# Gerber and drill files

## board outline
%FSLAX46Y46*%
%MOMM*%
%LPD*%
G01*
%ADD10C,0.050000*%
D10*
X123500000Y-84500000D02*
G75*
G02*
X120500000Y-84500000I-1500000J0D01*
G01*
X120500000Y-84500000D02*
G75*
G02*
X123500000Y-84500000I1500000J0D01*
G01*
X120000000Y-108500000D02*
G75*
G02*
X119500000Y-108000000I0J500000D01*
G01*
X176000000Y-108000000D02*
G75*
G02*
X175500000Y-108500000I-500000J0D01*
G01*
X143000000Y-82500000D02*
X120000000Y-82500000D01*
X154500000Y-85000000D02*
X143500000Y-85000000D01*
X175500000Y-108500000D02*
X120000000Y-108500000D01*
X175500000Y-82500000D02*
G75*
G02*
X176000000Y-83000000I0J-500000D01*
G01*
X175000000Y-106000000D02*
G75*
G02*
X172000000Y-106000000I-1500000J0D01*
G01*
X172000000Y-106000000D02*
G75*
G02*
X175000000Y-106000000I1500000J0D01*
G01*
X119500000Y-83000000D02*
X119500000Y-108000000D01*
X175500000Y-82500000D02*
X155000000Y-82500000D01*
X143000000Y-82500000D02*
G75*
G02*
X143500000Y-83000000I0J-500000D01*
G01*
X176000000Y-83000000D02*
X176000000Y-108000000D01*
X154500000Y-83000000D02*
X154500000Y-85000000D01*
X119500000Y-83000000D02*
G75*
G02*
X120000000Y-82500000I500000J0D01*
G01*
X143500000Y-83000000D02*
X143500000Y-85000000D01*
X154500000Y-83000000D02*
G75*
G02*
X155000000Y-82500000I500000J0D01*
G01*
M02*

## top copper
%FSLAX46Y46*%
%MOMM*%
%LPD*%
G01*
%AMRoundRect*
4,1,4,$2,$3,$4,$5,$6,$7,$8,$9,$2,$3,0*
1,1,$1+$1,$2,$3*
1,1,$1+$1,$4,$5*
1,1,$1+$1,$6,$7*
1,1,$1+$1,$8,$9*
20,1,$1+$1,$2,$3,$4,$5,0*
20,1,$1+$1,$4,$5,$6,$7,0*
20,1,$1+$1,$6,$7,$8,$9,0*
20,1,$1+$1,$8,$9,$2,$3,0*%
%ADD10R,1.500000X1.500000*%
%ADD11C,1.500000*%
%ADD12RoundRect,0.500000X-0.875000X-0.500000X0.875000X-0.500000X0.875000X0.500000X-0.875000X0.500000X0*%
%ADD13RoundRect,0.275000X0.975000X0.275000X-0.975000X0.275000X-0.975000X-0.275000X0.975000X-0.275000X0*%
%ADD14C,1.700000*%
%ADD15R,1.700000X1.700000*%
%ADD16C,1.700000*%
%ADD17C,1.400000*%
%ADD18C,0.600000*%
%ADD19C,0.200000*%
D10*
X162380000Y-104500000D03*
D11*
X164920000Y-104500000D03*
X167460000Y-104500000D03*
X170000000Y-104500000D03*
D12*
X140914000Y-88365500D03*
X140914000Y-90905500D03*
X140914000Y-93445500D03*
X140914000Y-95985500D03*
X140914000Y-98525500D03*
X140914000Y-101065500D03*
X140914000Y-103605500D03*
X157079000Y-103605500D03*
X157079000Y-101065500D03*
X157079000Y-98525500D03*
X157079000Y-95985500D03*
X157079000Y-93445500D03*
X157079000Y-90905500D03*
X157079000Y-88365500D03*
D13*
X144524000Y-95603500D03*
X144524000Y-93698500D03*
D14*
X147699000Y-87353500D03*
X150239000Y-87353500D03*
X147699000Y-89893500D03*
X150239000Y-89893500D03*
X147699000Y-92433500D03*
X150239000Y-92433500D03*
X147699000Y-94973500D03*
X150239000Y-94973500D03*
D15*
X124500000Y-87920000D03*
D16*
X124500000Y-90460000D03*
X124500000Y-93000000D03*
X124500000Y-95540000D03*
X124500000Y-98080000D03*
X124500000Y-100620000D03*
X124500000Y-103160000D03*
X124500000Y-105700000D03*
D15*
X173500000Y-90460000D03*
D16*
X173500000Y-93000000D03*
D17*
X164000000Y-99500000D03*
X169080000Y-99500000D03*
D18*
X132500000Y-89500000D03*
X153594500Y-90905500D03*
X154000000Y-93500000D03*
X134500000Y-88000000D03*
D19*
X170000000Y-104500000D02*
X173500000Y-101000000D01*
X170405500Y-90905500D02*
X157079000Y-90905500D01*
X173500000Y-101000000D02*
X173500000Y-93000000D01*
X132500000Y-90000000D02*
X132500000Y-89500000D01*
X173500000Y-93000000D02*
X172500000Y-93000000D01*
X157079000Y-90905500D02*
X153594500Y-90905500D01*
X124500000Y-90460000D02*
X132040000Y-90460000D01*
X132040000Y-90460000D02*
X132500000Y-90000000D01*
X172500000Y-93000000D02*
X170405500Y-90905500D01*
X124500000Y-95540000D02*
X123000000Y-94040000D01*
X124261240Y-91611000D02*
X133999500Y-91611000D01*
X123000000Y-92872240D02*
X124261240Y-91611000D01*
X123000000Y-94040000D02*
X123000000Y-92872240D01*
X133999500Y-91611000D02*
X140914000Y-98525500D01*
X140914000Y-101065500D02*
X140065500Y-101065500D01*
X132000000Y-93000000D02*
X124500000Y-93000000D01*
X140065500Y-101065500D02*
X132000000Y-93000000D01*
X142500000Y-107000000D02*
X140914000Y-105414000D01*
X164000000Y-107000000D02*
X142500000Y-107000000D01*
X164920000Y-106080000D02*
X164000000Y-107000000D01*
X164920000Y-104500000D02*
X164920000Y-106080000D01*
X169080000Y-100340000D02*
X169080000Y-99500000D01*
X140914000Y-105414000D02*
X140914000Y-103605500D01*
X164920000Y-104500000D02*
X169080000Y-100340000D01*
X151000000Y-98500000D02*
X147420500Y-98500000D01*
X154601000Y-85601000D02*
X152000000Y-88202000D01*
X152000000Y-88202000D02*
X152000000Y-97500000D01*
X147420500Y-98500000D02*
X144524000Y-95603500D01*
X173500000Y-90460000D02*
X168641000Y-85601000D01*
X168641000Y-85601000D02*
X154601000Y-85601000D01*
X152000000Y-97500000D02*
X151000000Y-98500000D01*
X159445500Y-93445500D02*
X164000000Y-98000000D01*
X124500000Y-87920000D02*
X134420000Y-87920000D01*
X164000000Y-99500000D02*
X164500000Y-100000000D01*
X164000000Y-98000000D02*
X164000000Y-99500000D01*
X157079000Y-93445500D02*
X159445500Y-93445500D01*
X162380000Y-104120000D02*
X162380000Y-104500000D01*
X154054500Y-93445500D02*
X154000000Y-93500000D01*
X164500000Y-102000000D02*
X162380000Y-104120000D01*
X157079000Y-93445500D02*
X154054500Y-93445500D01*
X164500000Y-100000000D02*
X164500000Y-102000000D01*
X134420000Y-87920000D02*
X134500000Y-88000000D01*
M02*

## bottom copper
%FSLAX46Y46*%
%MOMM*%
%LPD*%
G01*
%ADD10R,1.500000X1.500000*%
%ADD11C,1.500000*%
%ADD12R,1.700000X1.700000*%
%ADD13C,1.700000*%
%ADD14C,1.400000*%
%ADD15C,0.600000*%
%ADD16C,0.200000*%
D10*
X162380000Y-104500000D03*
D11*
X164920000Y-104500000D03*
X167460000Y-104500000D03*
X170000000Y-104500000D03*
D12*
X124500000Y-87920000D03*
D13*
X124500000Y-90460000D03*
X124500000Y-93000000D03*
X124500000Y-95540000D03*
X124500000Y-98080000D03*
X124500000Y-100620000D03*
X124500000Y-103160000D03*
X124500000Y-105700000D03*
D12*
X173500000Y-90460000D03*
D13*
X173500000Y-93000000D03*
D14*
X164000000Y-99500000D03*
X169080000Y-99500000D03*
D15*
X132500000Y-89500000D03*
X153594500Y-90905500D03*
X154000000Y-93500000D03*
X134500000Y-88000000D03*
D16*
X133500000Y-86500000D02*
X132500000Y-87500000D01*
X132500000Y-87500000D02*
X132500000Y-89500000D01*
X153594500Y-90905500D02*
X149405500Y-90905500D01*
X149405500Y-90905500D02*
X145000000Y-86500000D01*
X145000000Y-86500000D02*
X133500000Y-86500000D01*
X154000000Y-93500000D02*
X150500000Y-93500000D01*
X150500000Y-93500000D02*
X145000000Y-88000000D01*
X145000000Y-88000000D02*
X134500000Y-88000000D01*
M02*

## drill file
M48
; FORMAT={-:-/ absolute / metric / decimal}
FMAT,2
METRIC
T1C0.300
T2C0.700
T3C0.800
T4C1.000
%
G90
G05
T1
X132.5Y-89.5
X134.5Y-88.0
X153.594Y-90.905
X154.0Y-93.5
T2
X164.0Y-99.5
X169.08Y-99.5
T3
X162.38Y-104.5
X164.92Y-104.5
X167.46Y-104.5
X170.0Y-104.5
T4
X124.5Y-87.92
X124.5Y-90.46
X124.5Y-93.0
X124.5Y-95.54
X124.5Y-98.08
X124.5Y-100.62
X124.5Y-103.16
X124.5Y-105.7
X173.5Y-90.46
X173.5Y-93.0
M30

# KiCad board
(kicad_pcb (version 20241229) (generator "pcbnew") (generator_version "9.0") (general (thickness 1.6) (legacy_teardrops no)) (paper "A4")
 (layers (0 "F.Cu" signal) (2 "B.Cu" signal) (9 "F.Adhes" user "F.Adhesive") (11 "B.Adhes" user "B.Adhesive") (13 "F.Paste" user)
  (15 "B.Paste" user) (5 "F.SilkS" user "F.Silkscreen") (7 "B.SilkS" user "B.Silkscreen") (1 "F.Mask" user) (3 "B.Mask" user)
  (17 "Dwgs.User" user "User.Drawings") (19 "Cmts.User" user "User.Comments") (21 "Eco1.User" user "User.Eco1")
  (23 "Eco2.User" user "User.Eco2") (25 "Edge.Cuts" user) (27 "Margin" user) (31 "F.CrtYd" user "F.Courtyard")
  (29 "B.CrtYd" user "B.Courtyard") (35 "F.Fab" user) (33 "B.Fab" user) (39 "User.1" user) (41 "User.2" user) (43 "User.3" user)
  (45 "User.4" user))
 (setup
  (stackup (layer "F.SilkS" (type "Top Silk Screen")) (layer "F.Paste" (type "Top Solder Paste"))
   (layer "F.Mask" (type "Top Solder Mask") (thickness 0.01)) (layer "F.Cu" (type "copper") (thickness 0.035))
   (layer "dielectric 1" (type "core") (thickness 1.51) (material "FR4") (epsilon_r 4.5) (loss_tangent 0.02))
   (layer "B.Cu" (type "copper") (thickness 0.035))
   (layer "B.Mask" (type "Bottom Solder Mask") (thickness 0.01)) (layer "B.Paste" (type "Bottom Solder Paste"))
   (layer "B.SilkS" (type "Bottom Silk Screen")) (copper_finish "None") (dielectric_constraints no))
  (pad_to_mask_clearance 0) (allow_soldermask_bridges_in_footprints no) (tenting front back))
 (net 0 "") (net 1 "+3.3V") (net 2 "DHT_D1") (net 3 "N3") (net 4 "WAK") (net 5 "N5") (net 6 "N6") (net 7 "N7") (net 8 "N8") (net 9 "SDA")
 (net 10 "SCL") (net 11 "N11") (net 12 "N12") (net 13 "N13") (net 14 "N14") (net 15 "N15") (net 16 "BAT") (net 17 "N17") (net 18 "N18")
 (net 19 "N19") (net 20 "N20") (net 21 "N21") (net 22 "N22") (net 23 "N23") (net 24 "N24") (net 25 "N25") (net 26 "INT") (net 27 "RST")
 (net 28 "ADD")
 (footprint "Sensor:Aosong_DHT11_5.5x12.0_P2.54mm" (layer "F.Cu") (at 162.38 104.5 90)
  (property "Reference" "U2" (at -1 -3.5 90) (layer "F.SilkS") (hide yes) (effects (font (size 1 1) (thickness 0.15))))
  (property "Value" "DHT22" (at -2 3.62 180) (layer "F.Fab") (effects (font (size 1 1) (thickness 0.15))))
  (pad "1" thru_hole rect (at 0 0 90) (size 1.5 1.5) (drill 0.8) (layers "*.Cu" "*.Mask") (remove_unused_layers no) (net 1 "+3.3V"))
  (pad "2" thru_hole circle (at 0 2.54 90) (size 1.5 1.5) (drill 0.8) (layers "*.Cu" "*.Mask") (remove_unused_layers no) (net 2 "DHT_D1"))
  (pad "3" thru_hole circle (at 0 5.08 90) (size 1.5 1.5) (drill 0.8) (layers "*.Cu" "*.Mask") (remove_unused_layers no) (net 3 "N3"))
  (pad "4" thru_hole circle (at 0 7.62 90) (size 1.5 1.5) (drill 0.8) (layers "*.Cu" "*.Mask") (remove_unused_layers no) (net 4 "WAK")))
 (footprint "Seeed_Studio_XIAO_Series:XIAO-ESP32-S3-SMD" (layer "F.Cu") (at 140.079 106.4855)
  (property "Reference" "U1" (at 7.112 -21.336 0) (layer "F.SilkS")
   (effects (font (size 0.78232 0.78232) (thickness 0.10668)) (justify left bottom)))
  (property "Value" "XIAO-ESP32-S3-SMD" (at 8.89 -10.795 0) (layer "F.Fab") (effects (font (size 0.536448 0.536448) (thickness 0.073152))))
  (pad "1" smd roundrect (at 0.835 -18.12) (size 2.75 2) (layers "F.Cu" "F.Mask" "F.Paste") (roundrect_rratio 0.25) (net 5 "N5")
   (solder_mask_margin 0.0508) (thermal_bridge_angle 45))
  (pad "2" smd roundrect (at 0.835 -15.58) (size 2.75 2) (layers "F.Cu" "F.Mask" "F.Paste") (roundrect_rratio 0.25) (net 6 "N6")
   (solder_mask_margin 0.0508) (thermal_bridge_angle 45))
  (pad "3" smd roundrect (at 0.835 -13.04) (size 2.75 2) (layers "F.Cu" "F.Mask" "F.Paste") (roundrect_rratio 0.25) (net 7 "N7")
   (solder_mask_margin 0.0508) (thermal_bridge_angle 45))
  (pad "4" smd roundrect (at 0.835 -10.5) (size 2.75 2) (layers "F.Cu" "F.Mask" "F.Paste") (roundrect_rratio 0.25) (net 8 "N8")
   (solder_mask_margin 0.0508) (thermal_bridge_angle 45))
  (pad "5" smd roundrect (at 0.835 -7.96) (size 2.75 2) (layers "F.Cu" "F.Mask" "F.Paste") (roundrect_rratio 0.25) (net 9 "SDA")
   (solder_mask_margin 0.0508) (thermal_bridge_angle 45))
  (pad "6" smd roundrect (at 0.835 -5.42) (size 2.75 2) (layers "F.Cu" "F.Mask" "F.Paste") (roundrect_rratio 0.25) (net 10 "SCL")
   (solder_mask_margin 0.0508) (thermal_bridge_angle 45))
  (pad "7" smd roundrect (at 0.835 -2.88) (size 2.75 2) (layers "F.Cu" "F.Mask" "F.Paste") (roundrect_rratio 0.25) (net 2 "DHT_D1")
   (solder_mask_margin 0.0508) (thermal_bridge_angle 45))
  (pad "8" smd roundrect (at 17 -2.88) (size 2.75 2) (layers "F.Cu" "F.Mask" "F.Paste") (roundrect_rratio 0.25) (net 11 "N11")
   (solder_mask_margin 0.0508) (thermal_bridge_angle 45))
  (pad "9" smd roundrect (at 17 -5.42) (size 2.75 2) (layers "F.Cu" "F.Mask" "F.Paste") (roundrect_rratio 0.25) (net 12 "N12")
   (solder_mask_margin 0.0508) (thermal_bridge_angle 45))
  (pad "10" smd roundrect (at 17 -7.96) (size 2.75 2) (layers "F.Cu" "F.Mask" "F.Paste") (roundrect_rratio 0.25) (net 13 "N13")
   (solder_mask_margin 0.0508) (thermal_bridge_angle 45))
  (pad "11" smd roundrect (at 17 -10.5) (size 2.75 2) (layers "F.Cu" "F.Mask" "F.Paste") (roundrect_rratio 0.25) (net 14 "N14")
   (solder_mask_margin 0.0508) (thermal_bridge_angle 45))
  (pad "12" smd roundrect (at 17 -13.04) (size 2.75 2) (layers "F.Cu" "F.Mask" "F.Paste") (roundrect_rratio 0.25) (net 1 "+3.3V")
   (solder_mask_margin 0.0508) (thermal_bridge_angle 45))
  (pad "13" smd roundrect (at 17 -15.58) (size 2.75 2) (layers "F.Cu" "F.Mask" "F.Paste") (roundrect_rratio 0.25) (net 4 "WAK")
   (solder_mask_margin 0.0508) (thermal_bridge_angle 45))
  (pad "14" smd roundrect (at 17 -18.12) (size 2.75 2) (layers "F.Cu" "F.Mask" "F.Paste") (roundrect_rratio 0.25) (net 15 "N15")
   (solder_mask_margin 0.0508) (thermal_bridge_angle 45))
  (pad "15" smd roundrect (at 4.445 -10.882 180) (size 2.5 1.1) (layers "F.Cu" "F.Mask" "F.Paste") (roundrect_rratio 0.25) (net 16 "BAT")
   (solder_mask_margin 0.0508) (thermal_bridge_angle 45))
  (pad "16" smd roundrect (at 4.445 -12.787 180) (size 2.5 1.1) (layers "F.Cu" "F.Mask" "F.Paste") (roundrect_rratio 0.25) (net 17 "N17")
   (solder_mask_margin 0.0508) (thermal_bridge_angle 45))
  (pad "17" smd circle (at 7.62 -19.132) (size 1.7 1.7) (layers "F.Cu" "F.Mask" "F.Paste") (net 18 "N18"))
  (pad "18" smd circle (at 10.16 -19.132) (size 1.7 1.7) (layers "F.Cu" "F.Mask" "F.Paste") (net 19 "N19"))
  (pad "19" smd circle (at 7.62 -16.592) (size 1.7 1.7) (layers "F.Cu" "F.Mask" "F.Paste") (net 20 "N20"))
  (pad "20" smd circle (at 10.16 -16.592) (size 1.7 1.7) (layers "F.Cu" "F.Mask" "F.Paste") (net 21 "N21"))
  (pad "21" smd circle (at 7.62 -14.052) (size 1.7 1.7) (layers "F.Cu" "F.Mask" "F.Paste") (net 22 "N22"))
  (pad "22" smd circle (at 10.16 -14.052) (size 1.7 1.7) (layers "F.Cu" "F.Mask" "F.Paste") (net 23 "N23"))
  (pad "23" smd circle (at 7.62 -11.512) (size 1.7 1.7) (layers "F.Cu" "F.Mask" "F.Paste") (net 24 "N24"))
  (pad "24" smd circle (at 10.16 -11.512) (size 1.7 1.7) (layers "F.Cu" "F.Mask" "F.Paste") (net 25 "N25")))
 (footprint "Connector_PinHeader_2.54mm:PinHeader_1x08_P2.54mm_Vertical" (layer "F.Cu") (at 124.5 87.92)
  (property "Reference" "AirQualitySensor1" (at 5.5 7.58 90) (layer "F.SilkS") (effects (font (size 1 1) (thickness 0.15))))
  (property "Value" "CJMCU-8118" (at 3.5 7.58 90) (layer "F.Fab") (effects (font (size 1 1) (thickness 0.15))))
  (pad "1" thru_hole rect (at 0 0) (size 1.7 1.7) (drill 1) (layers "*.Cu" "*.Mask") (remove_unused_layers no) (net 1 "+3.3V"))
  (pad "2" thru_hole circle (at 0 2.54) (size 1.7 1.7) (drill 1) (layers "*.Cu" "*.Mask") (remove_unused_layers no) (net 4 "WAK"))
  (pad "3" thru_hole circle (at 0 5.08) (size 1.7 1.7) (drill 1) (layers "*.Cu" "*.Mask") (remove_unused_layers no) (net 10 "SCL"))
  (pad "4" thru_hole circle (at 0 7.62) (size 1.7 1.7) (drill 1) (layers "*.Cu" "*.Mask") (remove_unused_layers no) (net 9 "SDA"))
  (pad "5" thru_hole circle (at 0 10.16) (size 1.7 1.7) (drill 1) (layers "*.Cu" "*.Mask") (remove_unused_layers no) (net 4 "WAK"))
  (pad "6" thru_hole circle (at 0 12.7) (size 1.7 1.7) (drill 1) (layers "*.Cu" "*.Mask") (remove_unused_layers no) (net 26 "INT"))
  (pad "7" thru_hole circle (at 0 15.24) (size 1.7 1.7) (drill 1) (layers "*.Cu" "*.Mask") (remove_unused_layers no) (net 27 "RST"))
  (pad "8" thru_hole circle (at 0 17.78) (size 1.7 1.7) (drill 1) (layers "*.Cu" "*.Mask") (remove_unused_layers no) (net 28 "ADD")))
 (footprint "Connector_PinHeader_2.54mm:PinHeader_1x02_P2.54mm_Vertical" (layer "B.Cu") (at 173.5 90.46 180)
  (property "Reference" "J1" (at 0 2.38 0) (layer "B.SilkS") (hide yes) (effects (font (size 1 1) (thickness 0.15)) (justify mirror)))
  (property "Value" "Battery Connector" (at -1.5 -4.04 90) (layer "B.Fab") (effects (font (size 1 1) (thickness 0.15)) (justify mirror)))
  (pad "1" thru_hole rect (at 0 0 180) (size 1.7 1.7) (drill 1) (layers "*.Cu" "*.Mask") (remove_unused_layers no) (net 16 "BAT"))
  (pad "2" thru_hole circle (at 0 -2.54 180) (size 1.7 1.7) (drill 1) (layers "*.Cu" "*.Mask") (remove_unused_layers no) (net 4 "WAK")))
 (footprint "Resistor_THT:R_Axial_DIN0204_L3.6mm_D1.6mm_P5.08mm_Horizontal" (layer "B.Cu") (at 164 99.5)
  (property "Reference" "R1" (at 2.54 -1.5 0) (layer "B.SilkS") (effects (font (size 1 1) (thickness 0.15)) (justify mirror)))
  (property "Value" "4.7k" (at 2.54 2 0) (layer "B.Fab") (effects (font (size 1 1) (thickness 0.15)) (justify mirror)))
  (pad "1" thru_hole circle (at 0 0) (size 1.4 1.4) (drill 0.7) (layers "*.Cu" "*.Mask") (remove_unused_layers no) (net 1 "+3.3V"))
  (pad "2" thru_hole circle (at 5.08 0) (size 1.4 1.4) (drill 0.7) (layers "*.Cu" "*.Mask") (remove_unused_layers no) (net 2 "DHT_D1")))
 (gr_circle (center 122 84.5) (end 123.5 84.5) (stroke (width 0.05) (type solid)) (fill no) (layer "Edge.Cuts"))
 (gr_arc (start 120 108.5) (mid 119.646447 108.353553) (end 119.5 108) (stroke (width 0.05) (type default)) (layer "Edge.Cuts"))
 (gr_arc (start 176 108) (mid 175.853553 108.353553) (end 175.5 108.5) (stroke (width 0.05) (type default)) (layer "Edge.Cuts"))
 (gr_line (start 143 82.5) (end 120 82.5) (stroke (width 0.05) (type default)) (layer "Edge.Cuts"))
 (gr_line (start 154.5 85) (end 143.5 85) (stroke (width 0.05) (type default)) (layer "Edge.Cuts"))
 (gr_line (start 175.5 108.5) (end 120 108.5) (stroke (width 0.05) (type default)) (layer "Edge.Cuts"))
 (gr_arc (start 175.5 82.5) (mid 175.853553 82.646447) (end 176 83) (stroke (width 0.05) (type default)) (layer "Edge.Cuts"))
 (gr_circle (center 173.5 106) (end 175 106) (stroke (width 0.05) (type solid)) (fill no) (layer "Edge.Cuts"))
 (gr_line (start 119.5 83) (end 119.5 108) (stroke (width 0.05) (type default)) (layer "Edge.Cuts"))
 (gr_line (start 175.5 82.5) (end 155 82.5) (stroke (width 0.05) (type default)) (layer "Edge.Cuts"))
 (gr_arc (start 143 82.5) (mid 143.353553 82.646447) (end 143.5 83) (stroke (width 0.05) (type default)) (layer "Edge.Cuts"))
 (gr_line (start 176 83) (end 176 108) (stroke (width 0.05) (type default)) (layer "Edge.Cuts"))
 (gr_line (start 154.5 83) (end 154.5 85) (stroke (width 0.05) (type default)) (layer "Edge.Cuts"))
 (gr_arc (start 119.5 83) (mid 119.646447 82.646447) (end 120 82.5) (stroke (width 0.05) (type default)) (layer "Edge.Cuts"))
 (gr_line (start 143.5 83) (end 143.5 85) (stroke (width 0.05) (type default)) (layer "Edge.Cuts"))
 (gr_arc (start 154.5 83) (mid 154.646447 82.646447) (end 155 82.5) (stroke (width 0.05) (type default)) (layer "Edge.Cuts"))
 (segment (start 170 104.5) (end 173.5 101) (width 0.2) (layer "F.Cu") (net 4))
 (segment (start 170.4055 90.9055) (end 157.079 90.9055) (width 0.2) (layer "F.Cu") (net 4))
 (segment (start 173.5 101) (end 173.5 93) (width 0.2) (layer "F.Cu") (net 4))
 (segment (start 132.5 90) (end 132.5 89.5) (width 0.2) (layer "F.Cu") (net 4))
 (segment (start 173.5 93) (end 172.5 93) (width 0.2) (layer "F.Cu") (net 4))
 (segment (start 157.079 90.9055) (end 153.5945 90.9055) (width 0.2) (layer "F.Cu") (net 4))
 (segment (start 124.5 90.46) (end 132.04 90.46) (width 0.2) (layer "F.Cu") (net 4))
 (segment (start 132.04 90.46) (end 132.5 90) (width 0.2) (layer "F.Cu") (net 4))
 (segment (start 172.5 93) (end 170.4055 90.9055) (width 0.2) (layer "F.Cu") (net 4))
 (via (at 132.5 89.5) (size 0.6) (drill 0.3) (layers "F.Cu" "B.Cu") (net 4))
 (via (at 153.5945 90.9055) (size 0.6) (drill 0.3) (layers "F.Cu" "B.Cu") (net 4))
 (segment (start 133.5 86.5) (end 132.5 87.5) (width 0.2) (layer "B.Cu") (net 4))
 (segment (start 132.5 87.5) (end 132.5 89.5) (width 0.2) (layer "B.Cu") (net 4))
 (segment (start 153.5945 90.9055) (end 149.4055 90.9055) (width 0.2) (layer "B.Cu") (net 4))
 (segment (start 149.4055 90.9055) (end 145 86.5) (width 0.2) (layer "B.Cu") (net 4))
 (segment (start 145 86.5) (end 133.5 86.5) (width 0.2) (layer "B.Cu") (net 4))
 (segment (start 124.5 95.54) (end 123 94.04) (width 0.2) (layer "F.Cu") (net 9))
 (segment (start 124.26124 91.611) (end 133.9995 91.611) (width 0.2) (layer "F.Cu") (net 9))
 (segment (start 123 92.87224) (end 124.26124 91.611) (width 0.2) (layer "F.Cu") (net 9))
 (segment (start 123 94.04) (end 123 92.87224) (width 0.2) (layer "F.Cu") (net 9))
 (segment (start 133.9995 91.611) (end 140.914 98.5255) (width 0.2) (layer "F.Cu") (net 9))
 (segment (start 140.914 101.0655) (end 140.0655 101.0655) (width 0.2) (layer "F.Cu") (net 10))
 (segment (start 132 93) (end 124.5 93) (width 0.2) (layer "F.Cu") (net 10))
 (segment (start 140.0655 101.0655) (end 132 93) (width 0.2) (layer "F.Cu") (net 10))
 (segment (start 142.5 107) (end 140.914 105.414) (width 0.2) (layer "F.Cu") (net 2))
 (segment (start 164 107) (end 142.5 107) (width 0.2) (layer "F.Cu") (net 2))
 (segment (start 164.92 106.08) (end 164 107) (width 0.2) (layer "F.Cu") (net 2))
 (segment (start 164.92 104.5) (end 164.92 106.08) (width 0.2) (layer "F.Cu") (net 2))
 (segment (start 169.08 100.34) (end 169.08 99.5) (width 0.2) (layer "F.Cu") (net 2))
 (segment (start 140.914 105.414) (end 140.914 103.6055) (width 0.2) (layer "F.Cu") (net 2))
 (segment (start 164.92 104.5) (end 169.08 100.34) (width 0.2) (layer "F.Cu") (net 2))
 (segment (start 151 98.5) (end 147.4205 98.5) (width 0.2) (layer "F.Cu") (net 16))
 (segment (start 154.601 85.601) (end 152 88.202) (width 0.2) (layer "F.Cu") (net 16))
 (segment (start 152 88.202) (end 152 97.5) (width 0.2) (layer "F.Cu") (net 16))
 (segment (start 147.4205 98.5) (end 144.524 95.6035) (width 0.2) (layer "F.Cu") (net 16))
 (segment (start 173.5 90.46) (end 168.641 85.601) (width 0.2) (layer "F.Cu") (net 16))
 (segment (start 168.641 85.601) (end 154.601 85.601) (width 0.2) (layer "F.Cu") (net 16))
 (segment (start 152 97.5) (end 151 98.5) (width 0.2) (layer "F.Cu") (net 16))
 (segment (start 159.4455 93.4455) (end 164 98) (width 0.2) (layer "F.Cu") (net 1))
 (segment (start 124.5 87.92) (end 134.42 87.92) (width 0.2) (layer "F.Cu") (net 1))
 (segment (start 164 99.5) (end 164.5 100) (width 0.2) (layer "F.Cu") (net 1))
 (segment (start 164 98) (end 164 99.5) (width 0.2) (layer "F.Cu") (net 1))
 (segment (start 157.079 93.4455) (end 159.4455 93.4455) (width 0.2) (layer "F.Cu") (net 1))
 (segment (start 162.38 104.12) (end 162.38 104.5) (width 0.2) (layer "F.Cu") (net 1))
 (segment (start 154.0545 93.4455) (end 154 93.5) (width 0.2) (layer "F.Cu") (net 1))
 (segment (start 164.5 102) (end 162.38 104.12) (width 0.2) (layer "F.Cu") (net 1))
 (segment (start 157.079 93.4455) (end 154.0545 93.4455) (width 0.2) (layer "F.Cu") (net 1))
 (segment (start 164.5 100) (end 164.5 102) (width 0.2) (layer "F.Cu") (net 1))
 (segment (start 134.42 87.92) (end 134.5 88) (width 0.2) (layer "F.Cu") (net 1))
 (via (at 154 93.5) (size 0.6) (drill 0.3) (layers "F.Cu" "B.Cu") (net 1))
 (via (at 134.5 88) (size 0.6) (drill 0.3) (layers "F.Cu" "B.Cu") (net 1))
 (segment (start 154 93.5) (end 150.5 93.5) (width 0.2) (layer "B.Cu") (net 1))
 (segment (start 150.5 93.5) (end 145 88) (width 0.2) (layer "B.Cu") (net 1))
 (segment (start 145 88) (end 134.5 88) (width 0.2) (layer "B.Cu") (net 1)))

